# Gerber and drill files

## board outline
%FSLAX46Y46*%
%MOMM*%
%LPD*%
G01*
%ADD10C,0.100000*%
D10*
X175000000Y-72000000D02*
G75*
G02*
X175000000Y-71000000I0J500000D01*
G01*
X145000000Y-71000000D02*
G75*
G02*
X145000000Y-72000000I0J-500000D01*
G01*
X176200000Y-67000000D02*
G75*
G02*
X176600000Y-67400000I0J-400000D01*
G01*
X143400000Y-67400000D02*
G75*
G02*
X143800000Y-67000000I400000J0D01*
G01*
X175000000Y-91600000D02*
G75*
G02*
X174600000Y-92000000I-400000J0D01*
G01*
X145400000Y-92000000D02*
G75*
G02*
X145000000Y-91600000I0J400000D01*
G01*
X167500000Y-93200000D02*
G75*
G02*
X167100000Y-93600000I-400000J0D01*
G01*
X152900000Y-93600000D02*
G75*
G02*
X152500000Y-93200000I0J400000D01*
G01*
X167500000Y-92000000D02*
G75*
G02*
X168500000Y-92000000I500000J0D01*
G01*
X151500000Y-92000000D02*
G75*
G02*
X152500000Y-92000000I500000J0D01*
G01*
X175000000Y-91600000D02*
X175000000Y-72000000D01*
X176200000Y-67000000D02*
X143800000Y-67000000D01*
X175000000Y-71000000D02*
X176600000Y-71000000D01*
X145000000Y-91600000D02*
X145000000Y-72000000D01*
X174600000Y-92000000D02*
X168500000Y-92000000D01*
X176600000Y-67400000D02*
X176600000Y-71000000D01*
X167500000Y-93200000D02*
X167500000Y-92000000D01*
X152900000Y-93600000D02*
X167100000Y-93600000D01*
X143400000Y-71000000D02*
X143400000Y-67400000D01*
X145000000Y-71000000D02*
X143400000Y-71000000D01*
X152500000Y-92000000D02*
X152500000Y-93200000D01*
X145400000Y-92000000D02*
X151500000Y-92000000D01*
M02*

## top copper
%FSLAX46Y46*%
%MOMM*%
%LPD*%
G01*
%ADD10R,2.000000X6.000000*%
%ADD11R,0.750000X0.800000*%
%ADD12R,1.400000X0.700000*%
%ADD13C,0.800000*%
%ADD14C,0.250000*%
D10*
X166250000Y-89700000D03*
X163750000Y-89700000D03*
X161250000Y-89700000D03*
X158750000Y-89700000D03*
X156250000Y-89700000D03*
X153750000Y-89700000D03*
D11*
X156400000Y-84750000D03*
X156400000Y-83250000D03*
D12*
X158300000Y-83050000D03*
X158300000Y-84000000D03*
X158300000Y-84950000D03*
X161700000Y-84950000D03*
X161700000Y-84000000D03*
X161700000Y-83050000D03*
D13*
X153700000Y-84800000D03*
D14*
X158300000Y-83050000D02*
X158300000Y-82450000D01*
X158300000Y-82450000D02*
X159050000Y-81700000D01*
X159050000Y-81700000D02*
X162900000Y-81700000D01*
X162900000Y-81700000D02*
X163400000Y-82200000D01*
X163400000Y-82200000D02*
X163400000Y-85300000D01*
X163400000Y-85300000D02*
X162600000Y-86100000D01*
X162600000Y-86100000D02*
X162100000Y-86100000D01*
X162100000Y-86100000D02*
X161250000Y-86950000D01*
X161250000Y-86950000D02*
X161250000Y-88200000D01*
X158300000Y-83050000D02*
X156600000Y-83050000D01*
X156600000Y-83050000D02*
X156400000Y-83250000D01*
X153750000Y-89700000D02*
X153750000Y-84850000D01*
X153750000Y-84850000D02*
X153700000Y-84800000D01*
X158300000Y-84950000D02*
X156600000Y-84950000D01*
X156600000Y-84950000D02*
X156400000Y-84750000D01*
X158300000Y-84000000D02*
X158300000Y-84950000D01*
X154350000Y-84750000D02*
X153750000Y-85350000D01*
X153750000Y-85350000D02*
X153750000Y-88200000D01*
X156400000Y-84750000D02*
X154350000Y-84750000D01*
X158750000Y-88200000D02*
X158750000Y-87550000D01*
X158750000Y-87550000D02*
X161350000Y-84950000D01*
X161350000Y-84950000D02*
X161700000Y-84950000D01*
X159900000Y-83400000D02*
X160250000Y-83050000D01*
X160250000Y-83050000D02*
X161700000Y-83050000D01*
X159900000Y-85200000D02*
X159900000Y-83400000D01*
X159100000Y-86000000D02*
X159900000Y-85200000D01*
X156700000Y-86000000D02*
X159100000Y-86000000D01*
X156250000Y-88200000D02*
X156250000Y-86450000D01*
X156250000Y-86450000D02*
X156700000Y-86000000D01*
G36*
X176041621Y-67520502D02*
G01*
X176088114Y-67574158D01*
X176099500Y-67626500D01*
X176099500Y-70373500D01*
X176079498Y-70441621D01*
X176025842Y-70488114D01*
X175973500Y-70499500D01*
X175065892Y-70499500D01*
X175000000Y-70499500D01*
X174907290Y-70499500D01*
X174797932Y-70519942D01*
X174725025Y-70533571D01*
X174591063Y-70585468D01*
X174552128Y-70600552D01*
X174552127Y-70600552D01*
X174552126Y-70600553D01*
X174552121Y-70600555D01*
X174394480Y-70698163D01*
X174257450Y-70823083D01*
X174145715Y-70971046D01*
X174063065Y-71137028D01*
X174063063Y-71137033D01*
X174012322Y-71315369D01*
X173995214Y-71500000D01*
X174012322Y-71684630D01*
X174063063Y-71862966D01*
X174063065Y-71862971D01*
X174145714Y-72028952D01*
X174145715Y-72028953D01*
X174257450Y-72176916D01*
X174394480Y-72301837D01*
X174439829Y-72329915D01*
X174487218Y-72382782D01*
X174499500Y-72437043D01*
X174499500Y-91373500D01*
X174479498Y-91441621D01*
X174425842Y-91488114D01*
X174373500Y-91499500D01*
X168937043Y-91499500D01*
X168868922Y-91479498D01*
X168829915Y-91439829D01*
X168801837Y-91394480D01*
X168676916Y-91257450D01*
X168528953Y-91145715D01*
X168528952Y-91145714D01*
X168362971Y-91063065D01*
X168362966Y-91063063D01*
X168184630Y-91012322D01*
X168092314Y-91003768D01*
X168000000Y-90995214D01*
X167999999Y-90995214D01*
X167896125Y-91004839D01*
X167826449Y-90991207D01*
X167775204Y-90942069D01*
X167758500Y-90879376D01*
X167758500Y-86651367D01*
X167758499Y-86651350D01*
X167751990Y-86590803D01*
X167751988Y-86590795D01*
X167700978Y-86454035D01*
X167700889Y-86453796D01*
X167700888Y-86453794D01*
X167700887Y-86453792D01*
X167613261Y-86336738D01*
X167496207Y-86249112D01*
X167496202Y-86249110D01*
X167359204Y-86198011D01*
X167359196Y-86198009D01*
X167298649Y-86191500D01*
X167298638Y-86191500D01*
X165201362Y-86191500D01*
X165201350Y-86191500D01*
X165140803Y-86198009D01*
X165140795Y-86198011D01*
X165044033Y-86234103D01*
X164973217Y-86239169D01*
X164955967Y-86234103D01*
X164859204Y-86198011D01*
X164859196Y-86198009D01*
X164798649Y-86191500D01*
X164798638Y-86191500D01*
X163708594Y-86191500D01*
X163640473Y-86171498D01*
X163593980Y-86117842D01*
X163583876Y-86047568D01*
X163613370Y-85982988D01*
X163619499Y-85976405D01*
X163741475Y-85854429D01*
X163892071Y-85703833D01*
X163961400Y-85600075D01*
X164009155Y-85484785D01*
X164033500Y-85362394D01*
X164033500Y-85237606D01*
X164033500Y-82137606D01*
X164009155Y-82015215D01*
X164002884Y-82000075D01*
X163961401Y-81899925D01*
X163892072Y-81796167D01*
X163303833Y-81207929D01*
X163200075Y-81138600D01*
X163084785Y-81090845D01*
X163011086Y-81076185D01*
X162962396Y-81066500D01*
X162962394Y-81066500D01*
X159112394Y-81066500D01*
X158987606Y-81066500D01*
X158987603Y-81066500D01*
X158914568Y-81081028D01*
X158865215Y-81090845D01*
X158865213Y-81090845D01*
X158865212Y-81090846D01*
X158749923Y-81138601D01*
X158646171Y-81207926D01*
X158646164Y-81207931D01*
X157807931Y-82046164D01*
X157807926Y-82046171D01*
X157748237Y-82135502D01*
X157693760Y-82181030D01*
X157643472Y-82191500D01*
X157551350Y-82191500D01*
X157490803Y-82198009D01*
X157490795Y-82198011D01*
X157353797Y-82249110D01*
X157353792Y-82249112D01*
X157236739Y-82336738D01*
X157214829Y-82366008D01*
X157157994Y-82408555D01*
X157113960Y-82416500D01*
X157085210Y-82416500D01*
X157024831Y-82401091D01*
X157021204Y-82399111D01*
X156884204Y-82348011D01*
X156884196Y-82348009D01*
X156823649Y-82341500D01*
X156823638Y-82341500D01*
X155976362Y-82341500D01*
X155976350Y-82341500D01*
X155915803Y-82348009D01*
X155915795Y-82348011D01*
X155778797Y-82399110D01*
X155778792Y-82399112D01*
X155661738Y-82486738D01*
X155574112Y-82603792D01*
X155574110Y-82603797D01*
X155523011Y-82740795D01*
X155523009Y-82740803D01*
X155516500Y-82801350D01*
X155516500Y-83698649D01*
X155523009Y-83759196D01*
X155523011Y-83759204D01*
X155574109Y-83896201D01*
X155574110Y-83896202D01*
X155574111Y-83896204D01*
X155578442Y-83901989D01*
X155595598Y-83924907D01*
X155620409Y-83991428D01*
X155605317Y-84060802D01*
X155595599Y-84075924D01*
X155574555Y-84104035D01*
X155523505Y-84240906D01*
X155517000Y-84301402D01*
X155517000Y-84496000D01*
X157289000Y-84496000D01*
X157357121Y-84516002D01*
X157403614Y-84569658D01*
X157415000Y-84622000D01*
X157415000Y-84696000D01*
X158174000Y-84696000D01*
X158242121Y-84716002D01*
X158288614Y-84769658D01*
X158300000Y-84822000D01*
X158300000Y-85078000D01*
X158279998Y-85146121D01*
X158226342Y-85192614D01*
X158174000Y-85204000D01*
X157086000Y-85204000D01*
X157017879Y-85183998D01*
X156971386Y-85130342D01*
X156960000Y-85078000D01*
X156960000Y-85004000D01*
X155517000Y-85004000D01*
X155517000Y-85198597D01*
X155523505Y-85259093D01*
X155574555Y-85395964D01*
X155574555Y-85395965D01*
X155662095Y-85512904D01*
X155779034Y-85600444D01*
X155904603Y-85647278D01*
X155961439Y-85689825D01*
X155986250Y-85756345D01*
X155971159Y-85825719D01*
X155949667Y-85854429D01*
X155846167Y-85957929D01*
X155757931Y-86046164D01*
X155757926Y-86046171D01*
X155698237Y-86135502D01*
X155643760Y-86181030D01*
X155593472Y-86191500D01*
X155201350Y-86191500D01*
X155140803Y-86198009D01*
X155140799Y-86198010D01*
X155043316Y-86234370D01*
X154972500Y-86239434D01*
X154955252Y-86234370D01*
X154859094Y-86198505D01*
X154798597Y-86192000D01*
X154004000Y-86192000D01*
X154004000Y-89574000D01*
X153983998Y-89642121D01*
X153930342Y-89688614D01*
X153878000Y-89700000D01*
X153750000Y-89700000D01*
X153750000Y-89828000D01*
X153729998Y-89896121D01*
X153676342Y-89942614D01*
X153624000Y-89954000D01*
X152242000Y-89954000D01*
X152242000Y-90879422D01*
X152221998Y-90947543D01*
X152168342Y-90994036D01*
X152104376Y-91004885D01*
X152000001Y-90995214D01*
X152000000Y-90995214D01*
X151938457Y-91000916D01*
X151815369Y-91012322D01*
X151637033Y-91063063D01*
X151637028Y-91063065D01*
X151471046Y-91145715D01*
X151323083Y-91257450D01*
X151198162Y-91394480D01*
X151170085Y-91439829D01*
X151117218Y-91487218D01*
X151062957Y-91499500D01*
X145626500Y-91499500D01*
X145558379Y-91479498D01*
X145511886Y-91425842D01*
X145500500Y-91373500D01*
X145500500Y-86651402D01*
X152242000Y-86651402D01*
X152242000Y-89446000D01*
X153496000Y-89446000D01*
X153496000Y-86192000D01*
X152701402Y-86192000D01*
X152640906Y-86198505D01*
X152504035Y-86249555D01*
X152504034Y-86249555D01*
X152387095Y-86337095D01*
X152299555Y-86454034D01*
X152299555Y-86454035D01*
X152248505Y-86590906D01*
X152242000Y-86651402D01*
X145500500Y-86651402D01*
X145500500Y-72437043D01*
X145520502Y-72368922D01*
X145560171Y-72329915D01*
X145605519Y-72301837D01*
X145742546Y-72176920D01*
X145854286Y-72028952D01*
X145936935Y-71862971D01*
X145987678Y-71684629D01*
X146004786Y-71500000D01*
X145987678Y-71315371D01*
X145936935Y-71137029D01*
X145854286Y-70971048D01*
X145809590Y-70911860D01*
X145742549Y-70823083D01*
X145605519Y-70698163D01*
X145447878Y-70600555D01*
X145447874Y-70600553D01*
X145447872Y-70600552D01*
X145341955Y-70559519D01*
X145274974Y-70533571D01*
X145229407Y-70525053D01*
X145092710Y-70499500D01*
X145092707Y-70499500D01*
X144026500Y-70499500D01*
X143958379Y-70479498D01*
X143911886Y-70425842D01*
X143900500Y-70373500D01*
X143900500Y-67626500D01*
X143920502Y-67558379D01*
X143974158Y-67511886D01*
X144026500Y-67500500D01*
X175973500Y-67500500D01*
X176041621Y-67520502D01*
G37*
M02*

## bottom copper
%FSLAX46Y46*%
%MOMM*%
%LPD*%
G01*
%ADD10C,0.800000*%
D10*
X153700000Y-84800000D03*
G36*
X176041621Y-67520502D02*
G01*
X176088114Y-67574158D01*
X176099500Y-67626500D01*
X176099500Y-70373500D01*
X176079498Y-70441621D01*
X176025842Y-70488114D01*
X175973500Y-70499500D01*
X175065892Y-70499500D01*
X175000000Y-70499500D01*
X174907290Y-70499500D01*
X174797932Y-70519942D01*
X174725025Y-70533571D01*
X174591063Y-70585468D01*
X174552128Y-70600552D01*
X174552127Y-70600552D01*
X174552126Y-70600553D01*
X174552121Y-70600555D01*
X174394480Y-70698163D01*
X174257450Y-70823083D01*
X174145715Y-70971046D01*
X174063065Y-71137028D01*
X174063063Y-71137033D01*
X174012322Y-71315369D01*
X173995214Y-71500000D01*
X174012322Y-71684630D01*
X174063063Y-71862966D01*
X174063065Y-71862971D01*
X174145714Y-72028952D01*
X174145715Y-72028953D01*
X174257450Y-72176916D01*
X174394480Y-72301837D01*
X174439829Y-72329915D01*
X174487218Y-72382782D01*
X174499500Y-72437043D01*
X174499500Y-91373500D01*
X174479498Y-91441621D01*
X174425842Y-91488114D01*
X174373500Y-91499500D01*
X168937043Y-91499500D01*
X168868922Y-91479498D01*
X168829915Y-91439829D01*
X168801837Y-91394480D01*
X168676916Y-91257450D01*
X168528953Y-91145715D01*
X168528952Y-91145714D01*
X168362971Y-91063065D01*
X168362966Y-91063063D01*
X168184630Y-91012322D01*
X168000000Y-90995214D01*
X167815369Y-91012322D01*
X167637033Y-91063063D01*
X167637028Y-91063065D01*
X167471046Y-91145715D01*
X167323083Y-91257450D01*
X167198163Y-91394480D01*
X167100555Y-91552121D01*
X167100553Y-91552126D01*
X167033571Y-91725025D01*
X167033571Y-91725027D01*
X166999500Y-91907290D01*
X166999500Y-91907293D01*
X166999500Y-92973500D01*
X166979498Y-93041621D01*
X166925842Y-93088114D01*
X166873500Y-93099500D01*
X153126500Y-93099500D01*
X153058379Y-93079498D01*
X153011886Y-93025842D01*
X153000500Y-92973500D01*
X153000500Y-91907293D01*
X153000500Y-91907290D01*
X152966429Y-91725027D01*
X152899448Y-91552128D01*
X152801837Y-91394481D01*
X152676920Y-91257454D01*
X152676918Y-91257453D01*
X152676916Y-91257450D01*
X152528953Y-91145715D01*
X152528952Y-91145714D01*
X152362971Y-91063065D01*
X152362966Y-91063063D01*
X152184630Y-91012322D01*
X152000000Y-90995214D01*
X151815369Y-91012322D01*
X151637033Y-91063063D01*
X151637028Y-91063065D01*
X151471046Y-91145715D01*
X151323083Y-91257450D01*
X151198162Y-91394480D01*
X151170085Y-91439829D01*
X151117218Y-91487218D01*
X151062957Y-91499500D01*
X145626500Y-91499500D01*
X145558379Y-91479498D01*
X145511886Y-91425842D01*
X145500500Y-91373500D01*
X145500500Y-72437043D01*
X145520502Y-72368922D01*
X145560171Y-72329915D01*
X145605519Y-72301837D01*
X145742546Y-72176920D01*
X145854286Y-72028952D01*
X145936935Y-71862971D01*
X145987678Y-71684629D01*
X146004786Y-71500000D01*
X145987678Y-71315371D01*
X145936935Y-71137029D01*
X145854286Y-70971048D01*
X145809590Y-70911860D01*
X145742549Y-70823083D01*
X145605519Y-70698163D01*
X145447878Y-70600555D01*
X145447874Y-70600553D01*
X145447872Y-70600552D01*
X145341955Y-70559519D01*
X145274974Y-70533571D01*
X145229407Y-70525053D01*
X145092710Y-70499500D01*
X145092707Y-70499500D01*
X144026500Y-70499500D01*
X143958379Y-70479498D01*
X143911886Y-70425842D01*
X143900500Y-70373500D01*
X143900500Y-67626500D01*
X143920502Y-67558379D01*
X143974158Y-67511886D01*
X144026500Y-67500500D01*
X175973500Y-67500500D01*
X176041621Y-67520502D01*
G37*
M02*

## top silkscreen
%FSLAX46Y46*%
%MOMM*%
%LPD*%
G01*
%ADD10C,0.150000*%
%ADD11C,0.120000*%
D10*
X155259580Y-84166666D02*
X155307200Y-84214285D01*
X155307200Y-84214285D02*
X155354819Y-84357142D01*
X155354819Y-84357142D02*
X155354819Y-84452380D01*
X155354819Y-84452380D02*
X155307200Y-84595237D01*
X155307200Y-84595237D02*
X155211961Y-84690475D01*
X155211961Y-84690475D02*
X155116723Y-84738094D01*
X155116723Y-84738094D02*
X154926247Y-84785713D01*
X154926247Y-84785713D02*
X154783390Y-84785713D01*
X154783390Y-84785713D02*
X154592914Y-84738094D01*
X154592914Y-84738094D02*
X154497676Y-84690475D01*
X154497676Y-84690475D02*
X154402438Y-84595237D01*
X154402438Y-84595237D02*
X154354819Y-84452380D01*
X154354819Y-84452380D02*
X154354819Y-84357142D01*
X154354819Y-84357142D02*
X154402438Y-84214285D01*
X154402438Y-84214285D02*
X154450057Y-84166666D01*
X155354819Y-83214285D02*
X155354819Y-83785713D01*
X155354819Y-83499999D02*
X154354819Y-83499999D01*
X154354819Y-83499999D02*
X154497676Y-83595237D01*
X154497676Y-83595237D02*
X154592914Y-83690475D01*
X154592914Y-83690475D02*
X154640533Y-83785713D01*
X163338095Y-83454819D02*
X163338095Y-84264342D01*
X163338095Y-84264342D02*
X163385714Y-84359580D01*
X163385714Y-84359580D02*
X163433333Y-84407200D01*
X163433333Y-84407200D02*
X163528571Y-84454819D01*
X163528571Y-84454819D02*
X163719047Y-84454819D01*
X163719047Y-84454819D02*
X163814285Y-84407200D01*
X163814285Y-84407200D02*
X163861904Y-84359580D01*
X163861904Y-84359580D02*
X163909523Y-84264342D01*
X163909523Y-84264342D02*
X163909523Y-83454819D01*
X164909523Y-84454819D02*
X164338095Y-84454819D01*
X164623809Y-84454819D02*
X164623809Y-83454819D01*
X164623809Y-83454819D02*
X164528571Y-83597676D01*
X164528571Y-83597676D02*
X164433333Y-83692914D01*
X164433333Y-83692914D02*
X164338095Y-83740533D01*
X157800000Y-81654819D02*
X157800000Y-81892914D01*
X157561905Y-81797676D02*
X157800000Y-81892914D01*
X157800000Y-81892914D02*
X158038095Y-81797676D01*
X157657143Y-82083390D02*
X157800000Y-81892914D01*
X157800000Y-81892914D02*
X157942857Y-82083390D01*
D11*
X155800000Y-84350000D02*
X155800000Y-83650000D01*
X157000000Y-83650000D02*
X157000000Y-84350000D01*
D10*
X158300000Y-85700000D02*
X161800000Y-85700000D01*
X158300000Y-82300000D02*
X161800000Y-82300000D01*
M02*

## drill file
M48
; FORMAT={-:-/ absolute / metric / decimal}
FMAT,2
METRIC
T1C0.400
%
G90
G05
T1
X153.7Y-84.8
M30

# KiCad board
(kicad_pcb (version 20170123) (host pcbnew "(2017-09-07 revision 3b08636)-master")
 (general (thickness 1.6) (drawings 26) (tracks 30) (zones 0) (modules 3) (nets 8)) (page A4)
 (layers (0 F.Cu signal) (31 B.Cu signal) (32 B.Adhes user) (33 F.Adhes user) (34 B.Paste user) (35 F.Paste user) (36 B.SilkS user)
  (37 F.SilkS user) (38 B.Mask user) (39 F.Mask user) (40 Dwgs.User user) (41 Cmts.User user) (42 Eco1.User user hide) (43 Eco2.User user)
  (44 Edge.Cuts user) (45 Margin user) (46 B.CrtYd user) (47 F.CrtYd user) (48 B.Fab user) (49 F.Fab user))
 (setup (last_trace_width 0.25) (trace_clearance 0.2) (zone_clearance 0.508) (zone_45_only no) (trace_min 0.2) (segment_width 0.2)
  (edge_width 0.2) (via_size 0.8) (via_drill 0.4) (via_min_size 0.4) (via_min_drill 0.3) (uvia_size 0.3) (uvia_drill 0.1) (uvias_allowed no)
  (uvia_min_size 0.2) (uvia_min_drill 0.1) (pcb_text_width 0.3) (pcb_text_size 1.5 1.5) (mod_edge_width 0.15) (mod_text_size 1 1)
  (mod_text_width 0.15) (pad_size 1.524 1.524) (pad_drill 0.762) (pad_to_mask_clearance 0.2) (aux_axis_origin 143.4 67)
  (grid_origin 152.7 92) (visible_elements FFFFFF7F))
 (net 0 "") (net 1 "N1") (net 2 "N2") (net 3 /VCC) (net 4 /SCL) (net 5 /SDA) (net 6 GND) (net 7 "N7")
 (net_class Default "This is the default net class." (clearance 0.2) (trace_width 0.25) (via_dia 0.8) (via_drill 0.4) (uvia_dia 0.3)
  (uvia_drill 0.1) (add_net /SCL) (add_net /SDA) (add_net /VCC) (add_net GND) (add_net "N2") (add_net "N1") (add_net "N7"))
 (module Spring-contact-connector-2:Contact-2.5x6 (layer F.Cu) (at 160 90.7)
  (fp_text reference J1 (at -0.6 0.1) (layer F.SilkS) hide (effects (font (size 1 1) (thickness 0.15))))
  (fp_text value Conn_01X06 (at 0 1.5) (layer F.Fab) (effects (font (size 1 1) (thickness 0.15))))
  (pad 6 smd rect (at 6.25 -1) (size 2 6) (layers F.Cu F.Paste F.Mask) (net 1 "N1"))
  (pad 5 smd rect (at 3.75 -1) (size 2 6) (layers F.Cu F.Paste F.Mask) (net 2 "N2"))
  (pad 4 smd rect (at 1.25 -1) (size 2 6) (layers F.Cu F.Paste F.Mask) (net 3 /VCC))
  (pad 3 smd rect (at -1.25 -1) (size 2 6) (layers F.Cu F.Paste F.Mask) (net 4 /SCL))
  (pad 2 smd rect (at -3.75 -1) (size 2 6) (layers F.Cu F.Paste F.Mask) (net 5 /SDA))
  (pad 1 smd rect (at -6.25 -1) (size 2 6) (layers F.Cu F.Paste F.Mask) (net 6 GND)))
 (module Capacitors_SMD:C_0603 (layer F.Cu) (at 156.4 84 270)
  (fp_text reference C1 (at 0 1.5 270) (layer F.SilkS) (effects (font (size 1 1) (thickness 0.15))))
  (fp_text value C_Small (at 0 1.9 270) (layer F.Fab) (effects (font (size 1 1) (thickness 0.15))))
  (fp_line (start 0.35 0.6) (end -0.35 0.6) (layer F.SilkS) (width 0.12))
  (fp_line (start -0.35 -0.6) (end 0.35 -0.6) (layer F.SilkS) (width 0.12))
  (pad 2 smd rect (at 0.75 0 270) (size 0.8 0.75) (layers F.Cu F.Paste F.Mask) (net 6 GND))
  (pad 1 smd rect (at -0.75 0 270) (size 0.8 0.75) (layers F.Cu F.Paste F.Mask) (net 3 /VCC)))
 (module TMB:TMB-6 (layer F.Cu) (at 160 84)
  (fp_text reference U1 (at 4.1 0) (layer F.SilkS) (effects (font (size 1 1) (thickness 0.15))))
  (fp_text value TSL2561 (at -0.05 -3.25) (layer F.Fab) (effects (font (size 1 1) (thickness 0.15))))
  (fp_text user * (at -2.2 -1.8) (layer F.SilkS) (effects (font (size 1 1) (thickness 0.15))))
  (fp_line (start -1.7 1.7) (end 1.8 1.7) (layer F.SilkS) (width 0.15))
  (fp_line (start -1.7 -1.7) (end 1.8 -1.7) (layer F.SilkS) (width 0.15))
  (pad 1 smd rect (at -1.7 -0.95) (size 1.4 0.7) (layers F.Cu F.Paste F.Mask) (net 3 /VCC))
  (pad 2 smd rect (at -1.7 0) (size 1.4 0.7) (layers F.Cu F.Paste F.Mask) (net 6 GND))
  (pad 3 smd rect (at -1.7 0.95) (size 1.4 0.7) (layers F.Cu F.Paste F.Mask) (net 6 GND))
  (pad 4 smd rect (at 1.7 0.95) (size 1.4 0.7) (layers F.Cu F.Paste F.Mask) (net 4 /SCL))
  (pad 5 smd rect (at 1.7 0) (size 1.4 0.7) (layers F.Cu F.Paste F.Mask) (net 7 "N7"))
  (pad 6 smd rect (at 1.7 -0.95) (size 1.4 0.7) (layers F.Cu F.Paste F.Mask) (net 5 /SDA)))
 (gr_arc (start 175 71.5) (end 175 72) (angle 180) (layer Edge.Cuts) (width 0.1))
 (gr_arc (start 145 71.5) (end 145 71) (angle 180) (layer Edge.Cuts) (width 0.1))
 (gr_arc (start 176.2 67.4) (end 176.2 67) (angle 90) (layer Edge.Cuts) (width 0.1))
 (gr_arc (start 143.8 67.4) (end 143.4 67.4) (angle 90) (layer Edge.Cuts) (width 0.1))
 (gr_arc (start 174.6 91.6) (end 175 91.6) (angle 90) (layer Edge.Cuts) (width 0.1))
 (gr_arc (start 145.4 91.6) (end 145.4 92) (angle 90) (layer Edge.Cuts) (width 0.1))
 (gr_arc (start 167.1 93.2) (end 167.5 93.2) (angle 90) (layer Edge.Cuts) (width 0.1))
 (gr_arc (start 152.9 93.2) (end 152.9 93.6) (angle 90) (layer Edge.Cuts) (width 0.1))
 (gr_arc (start 168 92) (end 167.5 92) (angle 180) (layer Edge.Cuts) (width 0.1))
 (gr_arc (start 152 92) (end 151.5 92) (angle 180) (layer Edge.Cuts) (width 0.1))
 (gr_line (start 175 91.6) (end 175 72) (layer Edge.Cuts) (width 0.1))
 (gr_line (start 176.2 67) (end 143.8 67) (layer Edge.Cuts) (width 0.1))
 (gr_line (start 175 71) (end 176.6 71) (layer Edge.Cuts) (width 0.1))
 (gr_line (start 145 91.6) (end 145 72) (layer Edge.Cuts) (width 0.1))
 (gr_line (start 174.6 92) (end 168.5 92) (layer Edge.Cuts) (width 0.1))
 (gr_line (start 176.6 67.4) (end 176.6 71) (layer Edge.Cuts) (width 0.1))
 (gr_line (start 167.5 93.2) (end 167.5 92) (layer Edge.Cuts) (width 0.1))
 (gr_line (start 152.9 93.6) (end 167.1 93.6) (layer Edge.Cuts) (width 0.1))
 (gr_line (start 143.4 71) (end 143.4 67.4) (layer Edge.Cuts) (width 0.1))
 (gr_line (start 145 71) (end 143.4 71) (layer Edge.Cuts) (width 0.1))
 (gr_line (start 152.5 92) (end 152.5 93.2) (layer Edge.Cuts) (width 0.1))
 (gr_line (start 145.4 92) (end 151.5 92) (layer Edge.Cuts) (width 0.1))
 (segment (start 158.3 83.05) (end 158.3 82.45) (width 0.25) (layer F.Cu) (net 3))
 (segment (start 158.3 82.45) (end 159.05 81.7) (width 0.25) (layer F.Cu) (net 3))
 (segment (start 159.05 81.7) (end 162.9 81.7) (width 0.25) (layer F.Cu) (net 3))
 (segment (start 162.9 81.7) (end 163.4 82.2) (width 0.25) (layer F.Cu) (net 3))
 (segment (start 163.4 82.2) (end 163.4 85.3) (width 0.25) (layer F.Cu) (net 3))
 (segment (start 163.4 85.3) (end 162.6 86.1) (width 0.25) (layer F.Cu) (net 3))
 (segment (start 162.6 86.1) (end 162.1 86.1) (width 0.25) (layer F.Cu) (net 3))
 (segment (start 162.1 86.1) (end 161.25 86.95) (width 0.25) (layer F.Cu) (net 3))
 (segment (start 161.25 86.95) (end 161.25 88.2) (width 0.25) (layer F.Cu) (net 3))
 (segment (start 158.3 83.05) (end 156.6 83.05) (width 0.25) (layer F.Cu) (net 3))
 (segment (start 156.6 83.05) (end 156.4 83.25) (width 0.25) (layer F.Cu) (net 3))
 (segment (start 153.75 89.7) (end 153.75 84.85) (width 0.25) (layer F.Cu) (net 6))
 (segment (start 153.75 84.85) (end 153.7 84.8) (width 0.25) (layer F.Cu) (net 6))
 (via (at 153.7 84.8) (size 0.8) (drill 0.4) (layers F.Cu B.Cu) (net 6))
 (segment (start 158.3 84.95) (end 156.6 84.95) (width 0.25) (layer F.Cu) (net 6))
 (segment (start 156.6 84.95) (end 156.4 84.75) (width 0.25) (layer F.Cu) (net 6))
 (segment (start 158.3 84) (end 158.3 84.95) (width 0.25) (layer F.Cu) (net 6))
 (segment (start 154.35 84.75) (end 153.75 85.35) (width 0.25) (layer F.Cu) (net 6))
 (segment (start 153.75 85.35) (end 153.75 88.2) (width 0.25) (layer F.Cu) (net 6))
 (segment (start 156.4 84.75) (end 154.35 84.75) (width 0.25) (layer F.Cu) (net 6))
 (segment (start 158.75 88.2) (end 158.75 87.55) (width 0.25) (layer F.Cu) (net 4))
 (segment (start 158.75 87.55) (end 161.35 84.95) (width 0.25) (layer F.Cu) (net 4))
 (segment (start 161.35 84.95) (end 161.7 84.95) (width 0.25) (layer F.Cu) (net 4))
 (segment (start 159.9 83.4) (end 160.25 83.05) (width 0.25) (layer F.Cu) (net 5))
 (segment (start 160.25 83.05) (end 161.7 83.05) (width 0.25) (layer F.Cu) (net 5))
 (segment (start 159.9 85.2) (end 159.9 83.4) (width 0.25) (layer F.Cu) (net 5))
 (segment (start 159.1 86) (end 159.9 85.2) (width 0.25) (layer F.Cu) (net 5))
 (segment (start 156.7 86) (end 159.1 86) (width 0.25) (layer F.Cu) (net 5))
 (segment (start 156.25 88.2) (end 156.25 86.45) (width 0.25) (layer F.Cu) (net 5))
 (segment (start 156.25 86.45) (end 156.7 86) (width 0.25) (layer F.Cu) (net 5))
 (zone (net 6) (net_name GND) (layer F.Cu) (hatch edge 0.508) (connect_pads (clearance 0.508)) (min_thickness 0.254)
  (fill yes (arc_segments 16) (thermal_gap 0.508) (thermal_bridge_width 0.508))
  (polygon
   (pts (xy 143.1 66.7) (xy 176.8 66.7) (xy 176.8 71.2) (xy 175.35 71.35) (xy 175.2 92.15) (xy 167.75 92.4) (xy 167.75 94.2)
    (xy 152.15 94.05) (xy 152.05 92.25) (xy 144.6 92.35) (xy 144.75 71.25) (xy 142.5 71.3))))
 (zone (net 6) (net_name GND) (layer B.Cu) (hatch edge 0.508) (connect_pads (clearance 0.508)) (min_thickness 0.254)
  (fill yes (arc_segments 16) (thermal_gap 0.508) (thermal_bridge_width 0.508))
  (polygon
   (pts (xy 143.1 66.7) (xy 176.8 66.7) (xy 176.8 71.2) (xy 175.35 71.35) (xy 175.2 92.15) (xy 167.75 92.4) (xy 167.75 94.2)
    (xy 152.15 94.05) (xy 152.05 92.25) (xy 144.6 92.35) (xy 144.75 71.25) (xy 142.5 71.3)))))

